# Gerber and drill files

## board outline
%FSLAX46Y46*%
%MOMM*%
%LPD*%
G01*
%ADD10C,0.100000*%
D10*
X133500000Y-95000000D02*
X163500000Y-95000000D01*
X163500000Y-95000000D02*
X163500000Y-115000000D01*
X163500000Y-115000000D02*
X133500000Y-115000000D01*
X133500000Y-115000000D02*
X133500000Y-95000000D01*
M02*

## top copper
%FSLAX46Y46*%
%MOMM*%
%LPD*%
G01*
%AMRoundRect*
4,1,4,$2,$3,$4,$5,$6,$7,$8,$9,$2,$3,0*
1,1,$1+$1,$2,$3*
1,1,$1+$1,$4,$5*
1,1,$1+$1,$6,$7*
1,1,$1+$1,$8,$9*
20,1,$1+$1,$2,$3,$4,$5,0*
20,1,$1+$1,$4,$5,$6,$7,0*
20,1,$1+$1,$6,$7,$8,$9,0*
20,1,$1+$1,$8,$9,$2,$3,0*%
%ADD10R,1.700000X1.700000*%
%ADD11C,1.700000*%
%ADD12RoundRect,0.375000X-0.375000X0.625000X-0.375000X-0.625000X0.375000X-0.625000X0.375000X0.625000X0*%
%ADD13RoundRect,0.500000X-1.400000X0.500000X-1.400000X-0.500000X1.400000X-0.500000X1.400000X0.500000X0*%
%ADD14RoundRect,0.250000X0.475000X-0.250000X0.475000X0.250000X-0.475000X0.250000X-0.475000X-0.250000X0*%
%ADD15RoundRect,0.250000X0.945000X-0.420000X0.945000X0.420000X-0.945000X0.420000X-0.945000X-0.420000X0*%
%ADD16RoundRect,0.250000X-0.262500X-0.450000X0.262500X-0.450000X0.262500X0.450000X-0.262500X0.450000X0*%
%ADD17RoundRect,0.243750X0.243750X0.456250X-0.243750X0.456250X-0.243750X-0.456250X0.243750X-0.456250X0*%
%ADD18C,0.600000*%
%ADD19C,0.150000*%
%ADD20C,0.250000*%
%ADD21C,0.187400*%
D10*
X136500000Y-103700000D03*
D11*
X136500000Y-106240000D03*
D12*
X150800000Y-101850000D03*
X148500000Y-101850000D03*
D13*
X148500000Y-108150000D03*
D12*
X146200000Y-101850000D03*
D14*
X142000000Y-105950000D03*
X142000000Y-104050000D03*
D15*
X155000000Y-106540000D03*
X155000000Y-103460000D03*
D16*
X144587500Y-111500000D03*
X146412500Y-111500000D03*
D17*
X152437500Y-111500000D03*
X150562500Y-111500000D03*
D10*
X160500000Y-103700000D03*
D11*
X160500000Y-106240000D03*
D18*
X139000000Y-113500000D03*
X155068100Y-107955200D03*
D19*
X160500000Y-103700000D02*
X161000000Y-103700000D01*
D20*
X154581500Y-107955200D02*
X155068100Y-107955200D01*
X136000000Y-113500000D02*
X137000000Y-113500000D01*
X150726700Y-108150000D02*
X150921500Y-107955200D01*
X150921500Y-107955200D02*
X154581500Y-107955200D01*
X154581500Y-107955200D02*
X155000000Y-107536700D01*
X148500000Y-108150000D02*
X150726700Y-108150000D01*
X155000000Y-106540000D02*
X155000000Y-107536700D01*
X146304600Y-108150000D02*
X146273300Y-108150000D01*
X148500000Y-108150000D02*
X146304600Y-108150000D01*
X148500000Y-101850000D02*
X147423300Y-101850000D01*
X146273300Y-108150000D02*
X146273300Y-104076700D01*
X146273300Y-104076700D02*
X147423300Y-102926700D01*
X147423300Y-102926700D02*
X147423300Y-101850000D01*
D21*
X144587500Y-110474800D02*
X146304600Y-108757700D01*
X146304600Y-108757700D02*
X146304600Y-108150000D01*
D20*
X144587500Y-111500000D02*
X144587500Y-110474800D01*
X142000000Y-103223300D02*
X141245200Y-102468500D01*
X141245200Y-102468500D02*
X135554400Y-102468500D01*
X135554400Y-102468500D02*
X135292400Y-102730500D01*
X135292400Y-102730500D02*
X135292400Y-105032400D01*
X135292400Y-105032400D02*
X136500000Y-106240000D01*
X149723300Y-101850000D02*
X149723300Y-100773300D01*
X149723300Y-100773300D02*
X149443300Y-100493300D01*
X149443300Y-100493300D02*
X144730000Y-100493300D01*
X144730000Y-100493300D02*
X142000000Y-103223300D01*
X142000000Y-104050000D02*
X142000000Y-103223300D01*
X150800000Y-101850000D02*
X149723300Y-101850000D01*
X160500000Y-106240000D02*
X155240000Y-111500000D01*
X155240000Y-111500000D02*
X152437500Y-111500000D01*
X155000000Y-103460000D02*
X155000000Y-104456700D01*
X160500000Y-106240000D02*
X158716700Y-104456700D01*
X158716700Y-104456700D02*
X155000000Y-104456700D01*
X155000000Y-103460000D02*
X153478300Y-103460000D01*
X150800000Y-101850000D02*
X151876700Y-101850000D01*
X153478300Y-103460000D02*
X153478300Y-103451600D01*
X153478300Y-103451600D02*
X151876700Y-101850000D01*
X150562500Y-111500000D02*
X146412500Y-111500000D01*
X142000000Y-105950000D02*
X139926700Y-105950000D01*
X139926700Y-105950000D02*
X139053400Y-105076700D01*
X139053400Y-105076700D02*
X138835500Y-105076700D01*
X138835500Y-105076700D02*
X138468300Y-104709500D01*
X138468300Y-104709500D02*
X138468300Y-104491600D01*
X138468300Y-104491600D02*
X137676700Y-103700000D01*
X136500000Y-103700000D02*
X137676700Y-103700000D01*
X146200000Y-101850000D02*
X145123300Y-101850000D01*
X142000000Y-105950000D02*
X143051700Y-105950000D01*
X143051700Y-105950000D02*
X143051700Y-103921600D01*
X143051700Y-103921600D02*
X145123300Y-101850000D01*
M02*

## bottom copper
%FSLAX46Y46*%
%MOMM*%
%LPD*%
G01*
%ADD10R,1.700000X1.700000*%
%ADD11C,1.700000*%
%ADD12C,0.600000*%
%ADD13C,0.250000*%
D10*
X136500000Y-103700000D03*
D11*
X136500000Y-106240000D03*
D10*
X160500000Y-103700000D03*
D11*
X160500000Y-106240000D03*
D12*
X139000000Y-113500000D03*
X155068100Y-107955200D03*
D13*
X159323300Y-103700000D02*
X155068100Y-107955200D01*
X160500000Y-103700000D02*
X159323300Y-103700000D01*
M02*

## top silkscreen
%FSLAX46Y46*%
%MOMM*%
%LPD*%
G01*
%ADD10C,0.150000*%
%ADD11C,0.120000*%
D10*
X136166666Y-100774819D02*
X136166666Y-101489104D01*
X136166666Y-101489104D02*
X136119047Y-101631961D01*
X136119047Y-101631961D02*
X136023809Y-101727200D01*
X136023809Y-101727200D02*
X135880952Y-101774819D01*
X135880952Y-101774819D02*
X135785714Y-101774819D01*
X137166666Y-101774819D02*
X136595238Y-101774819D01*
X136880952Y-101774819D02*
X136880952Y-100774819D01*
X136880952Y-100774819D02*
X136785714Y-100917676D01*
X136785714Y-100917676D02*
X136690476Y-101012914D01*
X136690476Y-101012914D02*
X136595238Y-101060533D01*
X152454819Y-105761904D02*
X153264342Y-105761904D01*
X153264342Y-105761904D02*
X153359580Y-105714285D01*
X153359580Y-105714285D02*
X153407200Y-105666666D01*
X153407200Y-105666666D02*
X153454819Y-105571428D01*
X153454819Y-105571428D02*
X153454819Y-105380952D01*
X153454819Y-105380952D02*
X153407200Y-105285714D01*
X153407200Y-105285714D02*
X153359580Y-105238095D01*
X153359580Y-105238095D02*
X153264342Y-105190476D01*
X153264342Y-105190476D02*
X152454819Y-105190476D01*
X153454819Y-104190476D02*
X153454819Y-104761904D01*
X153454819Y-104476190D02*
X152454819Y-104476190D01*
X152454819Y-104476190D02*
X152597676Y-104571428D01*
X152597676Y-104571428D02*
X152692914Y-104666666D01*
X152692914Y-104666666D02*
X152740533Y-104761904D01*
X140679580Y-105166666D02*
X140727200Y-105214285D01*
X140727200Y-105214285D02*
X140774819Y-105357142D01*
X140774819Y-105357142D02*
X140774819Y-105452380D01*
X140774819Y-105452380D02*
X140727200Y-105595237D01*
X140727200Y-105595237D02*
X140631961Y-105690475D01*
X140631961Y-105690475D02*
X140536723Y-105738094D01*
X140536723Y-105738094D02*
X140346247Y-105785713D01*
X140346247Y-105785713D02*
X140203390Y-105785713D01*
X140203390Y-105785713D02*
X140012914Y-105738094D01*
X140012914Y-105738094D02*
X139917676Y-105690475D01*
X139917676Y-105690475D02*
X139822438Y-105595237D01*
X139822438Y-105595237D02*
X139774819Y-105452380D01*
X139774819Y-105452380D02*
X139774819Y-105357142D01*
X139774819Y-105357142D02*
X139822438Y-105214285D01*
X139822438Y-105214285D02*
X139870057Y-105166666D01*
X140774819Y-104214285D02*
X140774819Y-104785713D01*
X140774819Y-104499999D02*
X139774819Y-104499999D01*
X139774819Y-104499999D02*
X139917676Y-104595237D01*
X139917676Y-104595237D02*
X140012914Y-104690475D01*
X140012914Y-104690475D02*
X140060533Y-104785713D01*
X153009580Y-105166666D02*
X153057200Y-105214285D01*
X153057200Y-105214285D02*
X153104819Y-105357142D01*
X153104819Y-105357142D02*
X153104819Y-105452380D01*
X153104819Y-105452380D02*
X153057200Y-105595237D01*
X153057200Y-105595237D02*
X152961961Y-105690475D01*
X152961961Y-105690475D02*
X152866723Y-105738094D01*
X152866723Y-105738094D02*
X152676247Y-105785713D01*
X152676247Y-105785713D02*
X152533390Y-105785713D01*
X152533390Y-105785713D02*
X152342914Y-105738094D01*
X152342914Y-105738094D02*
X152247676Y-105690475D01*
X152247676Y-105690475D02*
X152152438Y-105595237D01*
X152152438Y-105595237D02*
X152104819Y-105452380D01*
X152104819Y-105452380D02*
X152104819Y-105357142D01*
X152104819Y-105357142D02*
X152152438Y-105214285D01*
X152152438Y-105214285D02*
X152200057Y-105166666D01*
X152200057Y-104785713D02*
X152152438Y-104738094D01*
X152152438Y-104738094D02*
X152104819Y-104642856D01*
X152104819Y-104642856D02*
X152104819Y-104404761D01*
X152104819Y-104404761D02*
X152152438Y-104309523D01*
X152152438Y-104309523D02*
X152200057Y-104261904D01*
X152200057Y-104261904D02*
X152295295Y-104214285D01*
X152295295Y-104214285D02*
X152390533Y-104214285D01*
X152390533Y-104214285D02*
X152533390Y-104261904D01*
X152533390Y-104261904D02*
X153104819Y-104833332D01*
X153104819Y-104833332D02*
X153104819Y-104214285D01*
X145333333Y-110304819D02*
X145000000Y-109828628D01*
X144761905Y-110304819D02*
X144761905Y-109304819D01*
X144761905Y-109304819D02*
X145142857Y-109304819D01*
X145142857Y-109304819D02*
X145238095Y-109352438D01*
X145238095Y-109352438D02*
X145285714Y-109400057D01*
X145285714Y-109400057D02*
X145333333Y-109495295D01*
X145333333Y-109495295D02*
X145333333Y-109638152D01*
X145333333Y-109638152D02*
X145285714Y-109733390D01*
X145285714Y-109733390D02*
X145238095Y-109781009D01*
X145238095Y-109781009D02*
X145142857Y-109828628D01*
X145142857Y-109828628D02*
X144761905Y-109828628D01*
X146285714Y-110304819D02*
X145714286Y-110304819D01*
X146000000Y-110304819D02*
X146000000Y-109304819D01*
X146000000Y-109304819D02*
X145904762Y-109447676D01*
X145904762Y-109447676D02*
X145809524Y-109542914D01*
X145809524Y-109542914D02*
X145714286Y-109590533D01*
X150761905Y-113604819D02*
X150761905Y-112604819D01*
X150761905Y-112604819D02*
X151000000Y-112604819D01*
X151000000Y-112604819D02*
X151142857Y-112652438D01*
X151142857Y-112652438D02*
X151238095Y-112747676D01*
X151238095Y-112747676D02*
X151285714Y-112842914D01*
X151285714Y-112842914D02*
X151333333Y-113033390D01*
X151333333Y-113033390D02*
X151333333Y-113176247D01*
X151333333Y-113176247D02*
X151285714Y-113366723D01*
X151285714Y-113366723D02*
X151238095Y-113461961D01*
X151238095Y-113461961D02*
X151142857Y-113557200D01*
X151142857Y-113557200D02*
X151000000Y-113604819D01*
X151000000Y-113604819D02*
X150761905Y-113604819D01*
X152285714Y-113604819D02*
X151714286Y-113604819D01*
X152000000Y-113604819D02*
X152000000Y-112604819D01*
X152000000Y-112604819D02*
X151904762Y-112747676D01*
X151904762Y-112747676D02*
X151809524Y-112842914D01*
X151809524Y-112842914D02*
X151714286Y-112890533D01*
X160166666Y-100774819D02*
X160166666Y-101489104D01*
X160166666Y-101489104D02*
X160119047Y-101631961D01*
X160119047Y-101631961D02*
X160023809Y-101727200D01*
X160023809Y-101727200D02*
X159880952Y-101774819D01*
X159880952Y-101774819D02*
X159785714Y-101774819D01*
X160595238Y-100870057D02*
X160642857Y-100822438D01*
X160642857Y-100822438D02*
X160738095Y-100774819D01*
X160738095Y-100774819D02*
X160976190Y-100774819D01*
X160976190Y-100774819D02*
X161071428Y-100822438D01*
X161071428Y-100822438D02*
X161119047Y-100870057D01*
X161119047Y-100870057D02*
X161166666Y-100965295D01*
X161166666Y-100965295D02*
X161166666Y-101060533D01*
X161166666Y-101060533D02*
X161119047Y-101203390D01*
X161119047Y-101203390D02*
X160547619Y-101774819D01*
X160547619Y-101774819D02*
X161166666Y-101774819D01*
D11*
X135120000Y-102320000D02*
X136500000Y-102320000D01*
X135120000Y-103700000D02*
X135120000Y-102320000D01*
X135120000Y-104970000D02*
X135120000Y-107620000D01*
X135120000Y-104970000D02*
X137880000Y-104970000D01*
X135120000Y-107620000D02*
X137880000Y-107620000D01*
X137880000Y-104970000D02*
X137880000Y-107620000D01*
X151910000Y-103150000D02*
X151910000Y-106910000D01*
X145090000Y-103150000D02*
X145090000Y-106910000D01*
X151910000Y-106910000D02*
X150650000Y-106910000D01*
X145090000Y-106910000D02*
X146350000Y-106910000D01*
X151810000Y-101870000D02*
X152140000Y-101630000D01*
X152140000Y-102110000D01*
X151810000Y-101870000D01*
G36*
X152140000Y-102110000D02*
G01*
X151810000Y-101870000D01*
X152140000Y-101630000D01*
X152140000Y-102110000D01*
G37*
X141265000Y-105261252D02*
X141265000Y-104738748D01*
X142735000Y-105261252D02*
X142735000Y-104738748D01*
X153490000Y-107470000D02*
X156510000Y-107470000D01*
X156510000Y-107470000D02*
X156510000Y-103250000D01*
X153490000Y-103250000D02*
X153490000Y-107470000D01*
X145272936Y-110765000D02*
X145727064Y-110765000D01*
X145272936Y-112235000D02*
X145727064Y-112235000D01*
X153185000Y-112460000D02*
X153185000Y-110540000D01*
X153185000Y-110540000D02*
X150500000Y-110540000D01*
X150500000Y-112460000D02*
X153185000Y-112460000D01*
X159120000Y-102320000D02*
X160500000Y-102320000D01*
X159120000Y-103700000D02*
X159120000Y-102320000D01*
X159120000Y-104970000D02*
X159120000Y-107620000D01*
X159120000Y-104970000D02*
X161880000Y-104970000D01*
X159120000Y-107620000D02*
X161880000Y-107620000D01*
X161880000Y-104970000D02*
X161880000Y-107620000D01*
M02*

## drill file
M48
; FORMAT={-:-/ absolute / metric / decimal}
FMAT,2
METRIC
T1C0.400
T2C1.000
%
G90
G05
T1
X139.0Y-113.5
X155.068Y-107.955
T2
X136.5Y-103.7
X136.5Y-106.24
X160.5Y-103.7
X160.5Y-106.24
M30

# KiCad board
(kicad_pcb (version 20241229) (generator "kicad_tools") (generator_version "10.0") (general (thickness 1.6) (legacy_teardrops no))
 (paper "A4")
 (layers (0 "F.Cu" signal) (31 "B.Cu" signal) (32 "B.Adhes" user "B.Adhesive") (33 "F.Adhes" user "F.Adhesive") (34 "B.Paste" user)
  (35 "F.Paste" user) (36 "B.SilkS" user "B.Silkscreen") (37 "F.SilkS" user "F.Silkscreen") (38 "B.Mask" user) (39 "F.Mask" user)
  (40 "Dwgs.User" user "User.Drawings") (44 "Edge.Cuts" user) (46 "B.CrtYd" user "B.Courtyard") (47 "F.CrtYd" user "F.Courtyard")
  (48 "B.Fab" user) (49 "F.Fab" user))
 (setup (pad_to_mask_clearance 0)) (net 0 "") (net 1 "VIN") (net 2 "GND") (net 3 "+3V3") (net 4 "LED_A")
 (gr_line (start 133.5 95) (end 163.5 95) (stroke (width 0.1) (type default)) (layer "Edge.Cuts"))
 (gr_line (start 163.5 95) (end 163.5 115) (stroke (width 0.1) (type default)) (layer "Edge.Cuts"))
 (gr_line (start 163.5 115) (end 133.5 115) (stroke (width 0.1) (type default)) (layer "Edge.Cuts"))
 (gr_line (start 133.5 115) (end 133.5 95) (stroke (width 0.1) (type default)) (layer "Edge.Cuts"))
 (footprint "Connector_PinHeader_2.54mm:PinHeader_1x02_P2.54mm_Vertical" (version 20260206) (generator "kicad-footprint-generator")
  (layer "F.Cu") (at 136.5 103.7)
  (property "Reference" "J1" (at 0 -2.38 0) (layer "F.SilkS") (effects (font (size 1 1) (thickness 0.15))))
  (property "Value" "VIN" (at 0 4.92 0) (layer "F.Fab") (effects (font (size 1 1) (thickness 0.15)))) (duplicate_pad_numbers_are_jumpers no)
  (fp_line (start -1.38 -1.38) (end 0 -1.38) (stroke (width 0.12) (type solid)) (layer "F.SilkS"))
  (fp_line (start -1.38 0) (end -1.38 -1.38) (stroke (width 0.12) (type solid)) (layer "F.SilkS"))
  (fp_line (start -1.38 1.27) (end -1.38 3.92) (stroke (width 0.12) (type solid)) (layer "F.SilkS"))
  (fp_line (start -1.38 1.27) (end 1.38 1.27) (stroke (width 0.12) (type solid)) (layer "F.SilkS"))
  (fp_line (start -1.38 3.92) (end 1.38 3.92) (stroke (width 0.12) (type solid)) (layer "F.SilkS"))
  (fp_line (start 1.38 1.27) (end 1.38 3.92) (stroke (width 0.12) (type solid)) (layer "F.SilkS"))
  (pad "1" thru_hole rect (at 0 0) (size 1.7 1.7) (drill 1) (layers "*.Cu" "*.Mask") (remove_unused_layers no) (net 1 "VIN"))
  (pad "2" thru_hole circle (at 0 2.54) (size 1.7 1.7) (drill 1) (layers "*.Cu" "*.Mask") (remove_unused_layers no) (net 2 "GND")))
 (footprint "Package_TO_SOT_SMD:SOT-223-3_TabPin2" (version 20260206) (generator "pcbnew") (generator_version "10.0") (layer "F.Cu")
  (at 148.5 105 -90)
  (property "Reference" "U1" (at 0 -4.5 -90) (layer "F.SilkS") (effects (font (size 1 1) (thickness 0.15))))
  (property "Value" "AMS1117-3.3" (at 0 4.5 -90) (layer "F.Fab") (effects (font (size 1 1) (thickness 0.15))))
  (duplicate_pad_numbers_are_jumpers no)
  (fp_line (start -1.85 -3.41) (end 1.91 -3.41) (stroke (width 0.12) (type solid)) (layer "F.SilkS"))
  (fp_line (start -1.85 3.41) (end 1.91 3.41) (stroke (width 0.12) (type solid)) (layer "F.SilkS"))
  (fp_line (start 1.91 -3.41) (end 1.91 -2.15) (stroke (width 0.12) (type solid)) (layer "F.SilkS"))
  (fp_line (start 1.91 3.41) (end 1.91 2.15) (stroke (width 0.12) (type solid)) (layer "F.SilkS"))
  (fp_poly
   (pts (xy -3.13 -3.31) (xy -3.37 -3.64) (xy -2.89 -3.64) (xy -3.13 -3.31)) (stroke (width 0.12) (type solid)) (fill yes) (layer "F.SilkS"))
  (pad "1" smd roundrect (at -3.15 -2.3 -90) (size 2 1.5) (layers "F.Cu" "F.Mask" "F.Paste") (roundrect_rratio 0.25) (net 2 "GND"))
  (pad "2" smd roundrect (at -3.15 0 -90) (size 2 1.5) (layers "F.Cu" "F.Mask" "F.Paste") (roundrect_rratio 0.25) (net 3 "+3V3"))
  (pad "2" smd roundrect (at 3.15 0 -90) (size 2 3.8) (layers "F.Cu" "F.Mask" "F.Paste") (roundrect_rratio 0.25) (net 3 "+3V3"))
  (pad "3" smd roundrect (at -3.15 2.3 -90) (size 2 1.5) (layers "F.Cu" "F.Mask" "F.Paste") (roundrect_rratio 0.25) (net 1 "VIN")))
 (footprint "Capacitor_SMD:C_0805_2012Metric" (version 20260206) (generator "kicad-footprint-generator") (layer "F.Cu") (at 142 105 90)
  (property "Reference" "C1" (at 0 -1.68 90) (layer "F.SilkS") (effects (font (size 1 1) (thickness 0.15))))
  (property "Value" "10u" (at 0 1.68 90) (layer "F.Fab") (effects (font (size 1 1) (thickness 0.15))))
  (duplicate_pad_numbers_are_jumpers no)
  (fp_line (start -0.261252 -0.735) (end 0.261252 -0.735) (stroke (width 0.12) (type solid)) (layer "F.SilkS"))
  (fp_line (start -0.261252 0.735) (end 0.261252 0.735) (stroke (width 0.12) (type solid)) (layer "F.SilkS"))
  (pad "1" smd roundrect (at -0.95 0 90) (size 1 1.45) (layers "F.Cu" "F.Mask" "F.Paste") (roundrect_rratio 0.25) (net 1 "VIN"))
  (pad "2" smd roundrect (at 0.95 0 90) (size 1 1.45) (layers "F.Cu" "F.Mask" "F.Paste") (roundrect_rratio 0.25) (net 2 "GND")))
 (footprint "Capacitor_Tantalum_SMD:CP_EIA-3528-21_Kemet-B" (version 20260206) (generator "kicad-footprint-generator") (layer "F.Cu")
  (at 155 105 90)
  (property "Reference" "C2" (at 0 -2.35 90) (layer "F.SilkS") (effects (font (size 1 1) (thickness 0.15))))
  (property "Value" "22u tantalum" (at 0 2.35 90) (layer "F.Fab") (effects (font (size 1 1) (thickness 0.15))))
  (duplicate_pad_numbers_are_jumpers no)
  (fp_line (start -2.47 -1.51) (end -2.47 1.51) (stroke (width 0.12) (type solid)) (layer "F.SilkS"))
  (fp_line (start -2.47 1.51) (end 1.75 1.51) (stroke (width 0.12) (type solid)) (layer "F.SilkS"))
  (fp_line (start 1.75 -1.51) (end -2.47 -1.51) (stroke (width 0.12) (type solid)) (layer "F.SilkS"))
  (pad "1" smd roundrect (at -1.54 0 90) (size 1.34 2.39) (layers "F.Cu" "F.Mask" "F.Paste") (roundrect_rratio 0.186567) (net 3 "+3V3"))
  (pad "2" smd roundrect (at 1.54 0 90) (size 1.34 2.39) (layers "F.Cu" "F.Mask" "F.Paste") (roundrect_rratio 0.186567) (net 2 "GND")))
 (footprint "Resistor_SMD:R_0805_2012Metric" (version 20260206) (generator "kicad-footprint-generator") (layer "F.Cu") (at 145.5 111.5)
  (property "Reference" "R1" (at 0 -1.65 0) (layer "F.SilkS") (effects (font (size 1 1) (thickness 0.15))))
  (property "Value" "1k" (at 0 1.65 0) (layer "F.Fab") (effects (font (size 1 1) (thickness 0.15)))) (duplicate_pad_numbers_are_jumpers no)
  (fp_line (start -0.227064 -0.735) (end 0.227064 -0.735) (stroke (width 0.12) (type solid)) (layer "F.SilkS"))
  (fp_line (start -0.227064 0.735) (end 0.227064 0.735) (stroke (width 0.12) (type solid)) (layer "F.SilkS"))
  (pad "1" smd roundrect (at -0.9125 0) (size 1.025 1.4) (layers "F.Cu" "F.Mask" "F.Paste") (roundrect_rratio 0.243902) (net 3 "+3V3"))
  (pad "2" smd roundrect (at 0.9125 0) (size 1.025 1.4) (layers "F.Cu" "F.Mask" "F.Paste") (roundrect_rratio 0.243902) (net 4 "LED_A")))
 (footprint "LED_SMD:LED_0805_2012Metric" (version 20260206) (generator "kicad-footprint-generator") (layer "F.Cu") (at 151.5 111.5 180)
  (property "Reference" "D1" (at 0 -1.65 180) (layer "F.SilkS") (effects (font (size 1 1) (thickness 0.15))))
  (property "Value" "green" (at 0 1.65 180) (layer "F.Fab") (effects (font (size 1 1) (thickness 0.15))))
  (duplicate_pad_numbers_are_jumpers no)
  (fp_line (start -1.685 -0.96) (end -1.685 0.96) (stroke (width 0.12) (type solid)) (layer "F.SilkS"))
  (fp_line (start -1.685 0.96) (end 1 0.96) (stroke (width 0.12) (type solid)) (layer "F.SilkS"))
  (fp_line (start 1 -0.96) (end -1.685 -0.96) (stroke (width 0.12) (type solid)) (layer "F.SilkS"))
  (pad "1" smd roundrect (at -0.9375 0 180) (size 0.975 1.4) (layers "F.Cu" "F.Mask" "F.Paste") (roundrect_rratio 0.25) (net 2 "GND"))
  (pad "2" smd roundrect (at 0.9375 0 180) (size 0.975 1.4) (layers "F.Cu" "F.Mask" "F.Paste") (roundrect_rratio 0.25) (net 4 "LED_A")))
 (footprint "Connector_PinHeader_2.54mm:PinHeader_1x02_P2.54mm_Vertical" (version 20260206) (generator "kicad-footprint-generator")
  (layer "F.Cu") (at 160.5 103.7)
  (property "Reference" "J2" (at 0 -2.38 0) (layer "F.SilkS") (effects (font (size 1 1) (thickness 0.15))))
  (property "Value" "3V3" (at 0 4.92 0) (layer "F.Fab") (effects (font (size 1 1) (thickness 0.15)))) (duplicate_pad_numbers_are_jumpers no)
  (fp_line (start -1.38 -1.38) (end 0 -1.38) (stroke (width 0.12) (type solid)) (layer "F.SilkS"))
  (fp_line (start -1.38 0) (end -1.38 -1.38) (stroke (width 0.12) (type solid)) (layer "F.SilkS"))
  (fp_line (start -1.38 1.27) (end -1.38 3.92) (stroke (width 0.12) (type solid)) (layer "F.SilkS"))
  (fp_line (start -1.38 1.27) (end 1.38 1.27) (stroke (width 0.12) (type solid)) (layer "F.SilkS"))
  (fp_line (start -1.38 3.92) (end 1.38 3.92) (stroke (width 0.12) (type solid)) (layer "F.SilkS"))
  (fp_line (start 1.38 1.27) (end 1.38 3.92) (stroke (width 0.12) (type solid)) (layer "F.SilkS"))
  (pad "1" thru_hole rect (at 0 0) (size 1.7 1.7) (drill 1) (layers "*.Cu" "*.Mask") (remove_unused_layers no) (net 3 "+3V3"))
  (pad "2" thru_hole circle (at 0 2.54) (size 1.7 1.7) (drill 1) (layers "*.Cu" "*.Mask") (remove_unused_layers no) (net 2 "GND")))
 (segment (start 160.5000 103.7000) (end 161.0000 103.7000) (width 0.15) (layer "F.Cu") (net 3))
 (segment (start 154.5815 107.9552) (end 155.0681 107.9552) (width 0.2500) (layer "F.Cu") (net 3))
 (segment (start 136.0000 113.5000) (end 137.0000 113.5000) (width 0.2500) (layer "F.Cu") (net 2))
 (segment (start 150.7267 108.1500) (end 150.9215 107.9552) (width 0.2500) (layer "F.Cu") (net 3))
 (segment (start 150.9215 107.9552) (end 154.5815 107.9552) (width 0.2500) (layer "F.Cu") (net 3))
 (segment (start 154.5815 107.9552) (end 155.0000 107.5367) (width 0.2500) (layer "F.Cu") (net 3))
 (segment (start 159.3233 103.7000) (end 155.0681 107.9552) (width 0.2500) (layer "B.Cu") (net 3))
 (segment (start 160.5000 103.7000) (end 159.3233 103.7000) (width 0.2500) (layer "B.Cu") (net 3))
 (segment (start 148.5000 108.1500) (end 150.7267 108.1500) (width 0.2500) (layer "F.Cu") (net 3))
 (segment (start 155.0000 106.5400) (end 155.0000 107.5367) (width 0.2500) (layer "F.Cu") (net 3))
 (segment (start 146.3046 108.1500) (end 146.2733 108.1500) (width 0.2500) (layer "F.Cu") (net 3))
 (segment (start 148.5000 108.1500) (end 146.3046 108.1500) (width 0.2500) (layer "F.Cu") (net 3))
 (segment (start 148.5000 101.8500) (end 147.4233 101.8500) (width 0.2500) (layer "F.Cu") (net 3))
 (segment (start 146.2733 108.1500) (end 146.2733 104.0767) (width 0.2500) (layer "F.Cu") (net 3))
 (segment (start 146.2733 104.0767) (end 147.4233 102.9267) (width 0.2500) (layer "F.Cu") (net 3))
 (segment (start 147.4233 102.9267) (end 147.4233 101.8500) (width 0.2500) (layer "F.Cu") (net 3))
 (segment (start 144.5875 110.4748) (end 146.3046 108.7577) (width 0.1874) (layer "F.Cu") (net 3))
 (segment (start 146.3046 108.7577) (end 146.3046 108.1500) (width 0.1874) (layer "F.Cu") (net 3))
 (segment (start 144.5875 111.5000) (end 144.5875 110.4748) (width 0.2500) (layer "F.Cu") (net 3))
 (segment (start 142.0000 103.2233) (end 141.2452 102.4685) (width 0.2500) (layer "F.Cu") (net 2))
 (segment (start 141.2452 102.4685) (end 135.5544 102.4685) (width 0.2500) (layer "F.Cu") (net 2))
 (segment (start 135.5544 102.4685) (end 135.2924 102.7305) (width 0.2500) (layer "F.Cu") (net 2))
 (segment (start 135.2924 102.7305) (end 135.2924 105.0324) (width 0.2500) (layer "F.Cu") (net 2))
 (segment (start 135.2924 105.0324) (end 136.5000 106.2400) (width 0.2500) (layer "F.Cu") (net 2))
 (segment (start 149.7233 101.8500) (end 149.7233 100.7733) (width 0.2500) (layer "F.Cu") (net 2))
 (segment (start 149.7233 100.7733) (end 149.4433 100.4933) (width 0.2500) (layer "F.Cu") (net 2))
 (segment (start 149.4433 100.4933) (end 144.7300 100.4933) (width 0.2500) (layer "F.Cu") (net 2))
 (segment (start 144.7300 100.4933) (end 142.0000 103.2233) (width 0.2500) (layer "F.Cu") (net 2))
 (segment (start 142.0000 104.0500) (end 142.0000 103.2233) (width 0.2500) (layer "F.Cu") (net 2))
 (segment (start 150.8000 101.8500) (end 149.7233 101.8500) (width 0.2500) (layer "F.Cu") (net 2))
 (segment (start 160.5000 106.2400) (end 155.2400 111.5000) (width 0.2500) (layer "F.Cu") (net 2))
 (segment (start 155.2400 111.5000) (end 152.4375 111.5000) (width 0.2500) (layer "F.Cu") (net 2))
 (segment (start 155.0000 103.4600) (end 155.0000 104.4567) (width 0.2500) (layer "F.Cu") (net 2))
 (segment (start 160.5000 106.2400) (end 158.7167 104.4567) (width 0.2500) (layer "F.Cu") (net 2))
 (segment (start 158.7167 104.4567) (end 155.0000 104.4567) (width 0.2500) (layer "F.Cu") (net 2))
 (segment (start 155.0000 103.4600) (end 153.4783 103.4600) (width 0.2500) (layer "F.Cu") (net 2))
 (segment (start 150.8000 101.8500) (end 151.8767 101.8500) (width 0.2500) (layer "F.Cu") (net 2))
 (segment (start 153.4783 103.4600) (end 153.4783 103.4516) (width 0.2500) (layer "F.Cu") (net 2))
 (segment (start 153.4783 103.4516) (end 151.8767 101.8500) (width 0.2500) (layer "F.Cu") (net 2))
 (segment (start 150.5625 111.5000) (end 146.4125 111.5000) (width 0.2500) (layer "F.Cu") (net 4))
 (segment (start 142.0000 105.9500) (end 139.9267 105.9500) (width 0.2500) (layer "F.Cu") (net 1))
 (segment (start 139.9267 105.9500) (end 139.0534 105.0767) (width 0.2500) (layer "F.Cu") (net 1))
 (segment (start 139.0534 105.0767) (end 138.8355 105.0767) (width 0.2500) (layer "F.Cu") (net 1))
 (segment (start 138.8355 105.0767) (end 138.4683 104.7095) (width 0.2500) (layer "F.Cu") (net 1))
 (segment (start 138.4683 104.7095) (end 138.4683 104.4916) (width 0.2500) (layer "F.Cu") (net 1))
 (segment (start 138.4683 104.4916) (end 137.6767 103.7000) (width 0.2500) (layer "F.Cu") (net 1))
 (segment (start 136.5000 103.7000) (end 137.6767 103.7000) (width 0.2500) (layer "F.Cu") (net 1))
 (segment (start 146.2000 101.8500) (end 145.1233 101.8500) (width 0.2500) (layer "F.Cu") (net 1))
 (segment (start 142.0000 105.9500) (end 143.0517 105.9500) (width 0.2500) (layer "F.Cu") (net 1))
 (segment (start 143.0517 105.9500) (end 143.0517 103.9216) (width 0.2500) (layer "F.Cu") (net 1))
 (segment (start 143.0517 103.9216) (end 145.1233 101.8500) (width 0.2500) (layer "F.Cu") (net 1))
 (via (at 139.0000 113.5000) (size 0.6000) (drill 0.4) (layers "F.Cu" "B.Cu") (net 2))
 (via (at 155.0681 107.9552) (size 0.6000) (drill 0.4) (layers "F.Cu" "B.Cu") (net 3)))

